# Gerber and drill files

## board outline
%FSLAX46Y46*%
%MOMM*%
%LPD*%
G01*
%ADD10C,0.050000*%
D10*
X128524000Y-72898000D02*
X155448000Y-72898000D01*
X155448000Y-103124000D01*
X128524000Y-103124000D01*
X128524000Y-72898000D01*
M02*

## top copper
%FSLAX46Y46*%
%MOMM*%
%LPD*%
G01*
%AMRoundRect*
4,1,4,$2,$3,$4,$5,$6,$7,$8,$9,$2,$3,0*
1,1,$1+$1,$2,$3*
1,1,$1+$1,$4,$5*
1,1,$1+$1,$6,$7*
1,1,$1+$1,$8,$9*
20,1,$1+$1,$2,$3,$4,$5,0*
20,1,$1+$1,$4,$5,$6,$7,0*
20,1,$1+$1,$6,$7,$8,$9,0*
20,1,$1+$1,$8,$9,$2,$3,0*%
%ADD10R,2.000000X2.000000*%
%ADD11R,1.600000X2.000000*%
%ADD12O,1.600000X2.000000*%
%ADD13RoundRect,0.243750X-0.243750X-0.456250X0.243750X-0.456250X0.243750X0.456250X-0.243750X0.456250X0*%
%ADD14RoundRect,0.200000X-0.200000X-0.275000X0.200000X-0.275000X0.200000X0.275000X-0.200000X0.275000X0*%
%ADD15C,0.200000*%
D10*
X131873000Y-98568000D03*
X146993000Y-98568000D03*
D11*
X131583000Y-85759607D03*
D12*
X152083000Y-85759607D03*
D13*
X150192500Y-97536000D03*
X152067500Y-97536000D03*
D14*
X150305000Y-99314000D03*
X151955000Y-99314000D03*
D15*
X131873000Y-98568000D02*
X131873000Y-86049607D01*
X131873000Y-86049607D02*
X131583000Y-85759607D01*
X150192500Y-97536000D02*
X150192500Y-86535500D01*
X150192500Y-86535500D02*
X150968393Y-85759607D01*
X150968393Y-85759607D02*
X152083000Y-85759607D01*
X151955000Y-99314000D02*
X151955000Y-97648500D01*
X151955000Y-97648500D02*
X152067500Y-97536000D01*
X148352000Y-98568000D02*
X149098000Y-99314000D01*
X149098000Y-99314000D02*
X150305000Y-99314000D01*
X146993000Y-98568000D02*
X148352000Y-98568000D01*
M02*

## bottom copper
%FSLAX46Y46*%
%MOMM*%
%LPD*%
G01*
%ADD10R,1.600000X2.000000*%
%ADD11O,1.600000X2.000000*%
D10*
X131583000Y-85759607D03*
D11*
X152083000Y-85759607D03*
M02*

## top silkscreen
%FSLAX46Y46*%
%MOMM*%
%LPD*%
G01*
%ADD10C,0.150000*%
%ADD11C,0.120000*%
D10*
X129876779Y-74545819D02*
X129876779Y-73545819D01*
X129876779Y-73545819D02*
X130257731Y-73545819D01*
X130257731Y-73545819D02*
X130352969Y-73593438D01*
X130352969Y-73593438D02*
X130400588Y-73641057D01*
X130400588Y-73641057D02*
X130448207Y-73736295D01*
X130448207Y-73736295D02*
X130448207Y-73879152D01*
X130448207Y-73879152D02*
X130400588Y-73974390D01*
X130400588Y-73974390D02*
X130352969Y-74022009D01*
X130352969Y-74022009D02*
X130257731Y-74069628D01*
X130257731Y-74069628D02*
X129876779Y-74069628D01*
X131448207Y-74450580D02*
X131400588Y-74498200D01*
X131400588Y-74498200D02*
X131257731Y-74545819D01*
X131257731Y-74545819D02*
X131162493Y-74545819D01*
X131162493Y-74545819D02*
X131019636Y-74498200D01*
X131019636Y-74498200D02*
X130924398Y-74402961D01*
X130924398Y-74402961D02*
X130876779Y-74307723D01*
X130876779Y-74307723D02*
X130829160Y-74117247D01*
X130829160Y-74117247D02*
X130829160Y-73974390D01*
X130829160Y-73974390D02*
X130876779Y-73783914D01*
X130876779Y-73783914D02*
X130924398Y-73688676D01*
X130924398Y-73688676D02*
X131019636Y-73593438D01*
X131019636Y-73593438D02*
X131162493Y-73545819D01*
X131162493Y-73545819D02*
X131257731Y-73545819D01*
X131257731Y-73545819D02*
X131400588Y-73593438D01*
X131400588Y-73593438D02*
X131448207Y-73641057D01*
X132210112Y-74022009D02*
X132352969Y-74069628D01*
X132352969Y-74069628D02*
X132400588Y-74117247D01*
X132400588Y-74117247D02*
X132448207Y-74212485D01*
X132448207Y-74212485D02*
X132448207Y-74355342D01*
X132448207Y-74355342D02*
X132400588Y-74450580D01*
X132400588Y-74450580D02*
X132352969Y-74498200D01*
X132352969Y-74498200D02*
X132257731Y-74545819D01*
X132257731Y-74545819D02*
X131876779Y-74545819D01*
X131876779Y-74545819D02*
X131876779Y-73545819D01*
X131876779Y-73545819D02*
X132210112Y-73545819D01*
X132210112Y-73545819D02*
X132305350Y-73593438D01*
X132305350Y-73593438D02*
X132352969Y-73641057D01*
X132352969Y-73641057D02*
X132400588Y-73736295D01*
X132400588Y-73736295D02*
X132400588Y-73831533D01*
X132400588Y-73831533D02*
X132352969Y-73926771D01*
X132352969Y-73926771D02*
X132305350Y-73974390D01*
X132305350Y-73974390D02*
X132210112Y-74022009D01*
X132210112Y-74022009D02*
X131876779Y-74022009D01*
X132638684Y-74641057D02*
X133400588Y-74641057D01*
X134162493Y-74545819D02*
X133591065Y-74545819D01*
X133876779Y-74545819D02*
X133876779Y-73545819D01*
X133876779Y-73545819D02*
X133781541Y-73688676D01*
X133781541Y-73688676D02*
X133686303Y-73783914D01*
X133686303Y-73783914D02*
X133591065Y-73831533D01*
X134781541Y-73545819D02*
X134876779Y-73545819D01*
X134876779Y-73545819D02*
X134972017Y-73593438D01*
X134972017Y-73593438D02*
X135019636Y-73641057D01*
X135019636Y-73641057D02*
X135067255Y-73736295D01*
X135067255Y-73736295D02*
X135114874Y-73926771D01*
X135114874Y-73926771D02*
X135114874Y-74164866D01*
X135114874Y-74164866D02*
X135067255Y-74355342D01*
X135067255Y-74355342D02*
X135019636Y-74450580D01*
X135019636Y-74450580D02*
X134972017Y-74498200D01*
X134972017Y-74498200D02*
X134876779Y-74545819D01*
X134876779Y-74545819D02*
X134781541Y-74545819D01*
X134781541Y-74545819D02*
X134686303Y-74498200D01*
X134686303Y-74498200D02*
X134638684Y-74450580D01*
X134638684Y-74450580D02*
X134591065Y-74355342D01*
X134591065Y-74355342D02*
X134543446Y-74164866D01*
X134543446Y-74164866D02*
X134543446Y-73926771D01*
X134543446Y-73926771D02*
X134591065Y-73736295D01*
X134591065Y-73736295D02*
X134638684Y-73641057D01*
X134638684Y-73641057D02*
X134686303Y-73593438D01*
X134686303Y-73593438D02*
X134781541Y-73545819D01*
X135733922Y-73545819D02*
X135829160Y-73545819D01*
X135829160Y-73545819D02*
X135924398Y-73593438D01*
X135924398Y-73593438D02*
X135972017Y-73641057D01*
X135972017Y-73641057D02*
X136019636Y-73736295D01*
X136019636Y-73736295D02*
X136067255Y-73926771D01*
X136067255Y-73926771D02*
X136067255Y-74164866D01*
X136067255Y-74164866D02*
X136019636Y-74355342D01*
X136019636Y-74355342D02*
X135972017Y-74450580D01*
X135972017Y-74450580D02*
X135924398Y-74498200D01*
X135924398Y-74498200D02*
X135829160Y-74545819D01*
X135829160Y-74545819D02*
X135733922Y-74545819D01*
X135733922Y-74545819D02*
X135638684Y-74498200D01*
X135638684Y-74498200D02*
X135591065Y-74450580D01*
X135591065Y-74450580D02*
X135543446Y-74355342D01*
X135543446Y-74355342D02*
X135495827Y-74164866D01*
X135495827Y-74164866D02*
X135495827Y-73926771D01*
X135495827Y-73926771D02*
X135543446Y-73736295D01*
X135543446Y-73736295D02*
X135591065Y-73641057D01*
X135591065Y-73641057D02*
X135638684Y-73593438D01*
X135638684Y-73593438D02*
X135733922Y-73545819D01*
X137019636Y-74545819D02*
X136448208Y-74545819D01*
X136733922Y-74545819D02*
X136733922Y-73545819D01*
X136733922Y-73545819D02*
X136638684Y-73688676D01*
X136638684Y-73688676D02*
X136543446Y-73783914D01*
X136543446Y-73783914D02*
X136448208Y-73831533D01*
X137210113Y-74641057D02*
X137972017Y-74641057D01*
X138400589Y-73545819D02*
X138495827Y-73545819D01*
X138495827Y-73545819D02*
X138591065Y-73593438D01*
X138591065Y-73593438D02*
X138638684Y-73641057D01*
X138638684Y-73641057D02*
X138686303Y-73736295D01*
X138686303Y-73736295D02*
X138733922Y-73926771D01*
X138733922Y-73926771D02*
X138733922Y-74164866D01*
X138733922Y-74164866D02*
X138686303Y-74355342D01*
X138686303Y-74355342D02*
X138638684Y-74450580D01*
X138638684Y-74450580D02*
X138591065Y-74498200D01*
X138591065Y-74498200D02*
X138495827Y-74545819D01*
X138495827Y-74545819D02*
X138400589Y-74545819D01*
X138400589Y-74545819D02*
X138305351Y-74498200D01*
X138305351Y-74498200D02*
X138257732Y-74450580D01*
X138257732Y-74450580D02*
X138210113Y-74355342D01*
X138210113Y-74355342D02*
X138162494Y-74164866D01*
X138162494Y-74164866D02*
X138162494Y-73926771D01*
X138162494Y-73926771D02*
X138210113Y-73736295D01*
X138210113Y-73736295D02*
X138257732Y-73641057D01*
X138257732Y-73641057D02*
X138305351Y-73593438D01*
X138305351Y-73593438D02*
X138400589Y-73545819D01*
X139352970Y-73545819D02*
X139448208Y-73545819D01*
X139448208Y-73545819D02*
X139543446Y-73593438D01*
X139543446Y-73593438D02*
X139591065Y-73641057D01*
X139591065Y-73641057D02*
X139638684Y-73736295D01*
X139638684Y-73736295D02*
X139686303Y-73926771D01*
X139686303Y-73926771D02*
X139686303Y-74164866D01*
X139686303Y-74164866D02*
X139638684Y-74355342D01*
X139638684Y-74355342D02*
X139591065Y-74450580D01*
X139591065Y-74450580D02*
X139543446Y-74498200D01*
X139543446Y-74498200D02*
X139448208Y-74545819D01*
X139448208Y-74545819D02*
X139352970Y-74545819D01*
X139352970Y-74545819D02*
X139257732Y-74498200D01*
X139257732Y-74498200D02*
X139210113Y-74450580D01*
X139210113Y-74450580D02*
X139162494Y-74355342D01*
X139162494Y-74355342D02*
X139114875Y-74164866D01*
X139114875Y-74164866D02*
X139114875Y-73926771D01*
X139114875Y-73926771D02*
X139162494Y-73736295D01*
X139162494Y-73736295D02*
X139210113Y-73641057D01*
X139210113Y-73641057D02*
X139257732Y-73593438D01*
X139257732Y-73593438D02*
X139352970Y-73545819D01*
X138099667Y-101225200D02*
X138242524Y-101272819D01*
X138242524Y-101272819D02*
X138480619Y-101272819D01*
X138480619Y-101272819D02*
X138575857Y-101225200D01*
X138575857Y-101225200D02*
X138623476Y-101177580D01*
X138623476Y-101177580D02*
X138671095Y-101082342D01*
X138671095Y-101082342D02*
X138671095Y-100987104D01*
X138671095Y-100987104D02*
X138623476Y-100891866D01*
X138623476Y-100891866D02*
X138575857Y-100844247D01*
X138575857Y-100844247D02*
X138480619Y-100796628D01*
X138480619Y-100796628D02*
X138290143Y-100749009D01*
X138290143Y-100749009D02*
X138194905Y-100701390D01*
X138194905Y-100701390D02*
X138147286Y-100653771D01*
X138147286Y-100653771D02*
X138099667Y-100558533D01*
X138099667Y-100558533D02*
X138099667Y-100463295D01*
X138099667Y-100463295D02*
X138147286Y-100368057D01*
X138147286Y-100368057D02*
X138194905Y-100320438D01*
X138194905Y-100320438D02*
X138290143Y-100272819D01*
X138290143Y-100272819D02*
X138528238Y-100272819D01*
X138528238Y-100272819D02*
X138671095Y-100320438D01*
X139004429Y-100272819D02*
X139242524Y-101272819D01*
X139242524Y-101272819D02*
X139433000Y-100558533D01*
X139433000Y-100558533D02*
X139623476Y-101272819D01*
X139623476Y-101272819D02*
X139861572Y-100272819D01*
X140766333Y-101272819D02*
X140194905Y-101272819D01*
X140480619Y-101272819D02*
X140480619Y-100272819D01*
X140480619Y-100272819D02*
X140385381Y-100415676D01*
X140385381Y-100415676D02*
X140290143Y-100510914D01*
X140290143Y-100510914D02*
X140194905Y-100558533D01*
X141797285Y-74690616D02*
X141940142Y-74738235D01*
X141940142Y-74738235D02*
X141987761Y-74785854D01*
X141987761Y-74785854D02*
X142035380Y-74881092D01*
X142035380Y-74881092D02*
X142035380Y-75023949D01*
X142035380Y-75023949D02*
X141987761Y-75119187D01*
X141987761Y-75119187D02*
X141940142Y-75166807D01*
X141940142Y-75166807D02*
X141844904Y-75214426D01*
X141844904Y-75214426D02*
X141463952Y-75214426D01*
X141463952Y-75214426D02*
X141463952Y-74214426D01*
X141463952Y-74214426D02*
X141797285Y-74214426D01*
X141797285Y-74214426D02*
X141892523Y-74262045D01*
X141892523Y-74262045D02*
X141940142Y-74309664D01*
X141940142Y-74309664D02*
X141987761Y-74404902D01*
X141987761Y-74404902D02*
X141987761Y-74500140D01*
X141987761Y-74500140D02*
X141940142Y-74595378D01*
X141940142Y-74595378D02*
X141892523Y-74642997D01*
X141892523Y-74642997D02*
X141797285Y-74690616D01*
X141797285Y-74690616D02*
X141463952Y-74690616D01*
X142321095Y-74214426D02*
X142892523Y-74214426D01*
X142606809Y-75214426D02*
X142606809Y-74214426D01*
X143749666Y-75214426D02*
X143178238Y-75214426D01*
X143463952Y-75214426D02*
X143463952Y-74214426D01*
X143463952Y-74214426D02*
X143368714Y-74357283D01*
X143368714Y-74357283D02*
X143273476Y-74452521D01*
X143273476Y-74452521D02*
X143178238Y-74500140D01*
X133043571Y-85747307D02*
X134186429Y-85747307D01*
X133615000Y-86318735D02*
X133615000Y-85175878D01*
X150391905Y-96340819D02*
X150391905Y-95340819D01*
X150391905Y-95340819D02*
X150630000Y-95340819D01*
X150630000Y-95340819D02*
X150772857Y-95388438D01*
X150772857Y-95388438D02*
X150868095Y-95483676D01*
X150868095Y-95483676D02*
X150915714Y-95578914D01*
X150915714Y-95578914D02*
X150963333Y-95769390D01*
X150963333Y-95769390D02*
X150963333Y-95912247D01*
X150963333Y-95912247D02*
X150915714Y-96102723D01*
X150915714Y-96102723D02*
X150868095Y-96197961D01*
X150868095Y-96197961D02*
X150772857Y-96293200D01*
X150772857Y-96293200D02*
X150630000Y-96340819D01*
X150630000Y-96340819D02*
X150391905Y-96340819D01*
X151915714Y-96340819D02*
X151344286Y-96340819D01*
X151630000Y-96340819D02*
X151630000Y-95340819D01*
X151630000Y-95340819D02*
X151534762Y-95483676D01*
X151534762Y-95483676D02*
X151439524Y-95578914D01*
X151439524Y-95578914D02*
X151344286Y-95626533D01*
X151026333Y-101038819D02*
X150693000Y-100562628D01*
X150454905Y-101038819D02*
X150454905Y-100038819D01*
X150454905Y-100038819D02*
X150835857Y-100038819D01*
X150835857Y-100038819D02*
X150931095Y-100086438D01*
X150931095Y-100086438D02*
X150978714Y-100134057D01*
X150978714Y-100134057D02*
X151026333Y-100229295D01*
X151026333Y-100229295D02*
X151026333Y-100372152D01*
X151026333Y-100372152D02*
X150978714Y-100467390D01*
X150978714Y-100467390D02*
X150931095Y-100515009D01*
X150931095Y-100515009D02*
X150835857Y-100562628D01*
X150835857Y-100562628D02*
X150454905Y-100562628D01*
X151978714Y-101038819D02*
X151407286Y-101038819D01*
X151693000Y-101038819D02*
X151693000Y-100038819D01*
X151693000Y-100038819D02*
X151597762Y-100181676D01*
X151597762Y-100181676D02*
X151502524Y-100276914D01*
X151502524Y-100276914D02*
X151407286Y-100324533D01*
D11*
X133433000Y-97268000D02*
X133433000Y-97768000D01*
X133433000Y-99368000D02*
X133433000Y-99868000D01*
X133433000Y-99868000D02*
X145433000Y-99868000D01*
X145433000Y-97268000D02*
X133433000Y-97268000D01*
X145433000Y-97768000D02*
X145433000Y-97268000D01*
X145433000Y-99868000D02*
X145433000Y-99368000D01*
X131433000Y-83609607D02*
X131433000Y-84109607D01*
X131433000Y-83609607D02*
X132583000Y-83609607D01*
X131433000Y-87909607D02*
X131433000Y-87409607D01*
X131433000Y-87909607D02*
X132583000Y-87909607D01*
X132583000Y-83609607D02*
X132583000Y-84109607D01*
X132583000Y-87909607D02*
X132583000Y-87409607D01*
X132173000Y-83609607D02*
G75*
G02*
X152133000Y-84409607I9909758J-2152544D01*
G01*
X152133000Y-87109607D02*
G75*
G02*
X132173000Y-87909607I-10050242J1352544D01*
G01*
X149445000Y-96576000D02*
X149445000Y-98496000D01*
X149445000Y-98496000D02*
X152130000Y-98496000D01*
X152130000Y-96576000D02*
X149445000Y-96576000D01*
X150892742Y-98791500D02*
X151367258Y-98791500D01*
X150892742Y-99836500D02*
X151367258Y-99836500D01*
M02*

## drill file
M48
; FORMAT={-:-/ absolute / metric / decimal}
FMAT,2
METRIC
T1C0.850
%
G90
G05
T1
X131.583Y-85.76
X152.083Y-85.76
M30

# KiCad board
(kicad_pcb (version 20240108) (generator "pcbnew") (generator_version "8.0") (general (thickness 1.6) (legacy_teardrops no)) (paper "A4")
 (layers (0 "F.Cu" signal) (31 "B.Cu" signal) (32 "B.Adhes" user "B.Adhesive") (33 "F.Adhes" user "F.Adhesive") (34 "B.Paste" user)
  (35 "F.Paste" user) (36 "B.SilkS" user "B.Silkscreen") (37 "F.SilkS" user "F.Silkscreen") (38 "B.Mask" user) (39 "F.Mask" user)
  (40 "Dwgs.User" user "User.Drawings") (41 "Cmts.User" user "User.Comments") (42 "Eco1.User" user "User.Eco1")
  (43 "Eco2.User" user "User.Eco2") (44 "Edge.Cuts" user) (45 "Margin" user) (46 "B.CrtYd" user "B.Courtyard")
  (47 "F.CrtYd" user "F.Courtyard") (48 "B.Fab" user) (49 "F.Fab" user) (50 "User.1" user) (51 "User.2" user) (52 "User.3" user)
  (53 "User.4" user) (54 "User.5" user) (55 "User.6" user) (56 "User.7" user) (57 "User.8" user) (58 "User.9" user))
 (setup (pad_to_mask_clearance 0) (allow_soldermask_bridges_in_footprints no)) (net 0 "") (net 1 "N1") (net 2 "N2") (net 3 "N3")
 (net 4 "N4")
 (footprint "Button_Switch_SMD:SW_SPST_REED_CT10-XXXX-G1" (layer "F.Cu") (at 139.433 98.568)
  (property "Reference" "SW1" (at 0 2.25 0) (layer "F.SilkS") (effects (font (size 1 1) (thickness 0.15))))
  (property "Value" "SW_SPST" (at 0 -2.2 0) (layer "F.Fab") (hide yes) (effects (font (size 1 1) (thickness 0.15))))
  (fp_line (start -6 -1.3) (end -6 -0.8) (stroke (width 0.12) (type solid)) (layer "F.SilkS"))
  (fp_line (start -6 0.8) (end -6 1.3) (stroke (width 0.12) (type solid)) (layer "F.SilkS"))
  (fp_line (start -6 1.3) (end 6 1.3) (stroke (width 0.12) (type solid)) (layer "F.SilkS"))
  (fp_line (start 6 -1.3) (end -6 -1.3) (stroke (width 0.12) (type solid)) (layer "F.SilkS"))
  (fp_line (start 6 -0.8) (end 6 -1.3) (stroke (width 0.12) (type solid)) (layer "F.SilkS"))
  (fp_line (start 6 1.3) (end 6 0.8) (stroke (width 0.12) (type solid)) (layer "F.SilkS"))
  (pad "1" smd rect (at -7.56 0) (size 2 2) (layers "F.Cu" "F.Paste" "F.Mask") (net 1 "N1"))
  (pad "2" smd rect (at 7.56 0) (size 2 2) (layers "F.Cu" "F.Paste" "F.Mask") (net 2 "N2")))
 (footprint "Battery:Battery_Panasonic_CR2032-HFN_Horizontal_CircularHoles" (layer "F.Cu") (at 131.583 85.759607)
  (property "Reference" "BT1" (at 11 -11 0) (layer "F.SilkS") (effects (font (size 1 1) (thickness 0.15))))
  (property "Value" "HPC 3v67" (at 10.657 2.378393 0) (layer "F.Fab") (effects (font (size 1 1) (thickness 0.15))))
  (fp_line (start -0.15 -2.15) (end -0.15 -1.65) (stroke (width 0.12) (type default)) (layer "F.SilkS"))
  (fp_line (start -0.15 -2.15) (end 1 -2.15) (stroke (width 0.12) (type default)) (layer "F.SilkS"))
  (fp_line (start -0.15 2.15) (end -0.15 1.65) (stroke (width 0.12) (type default)) (layer "F.SilkS"))
  (fp_line (start -0.15 2.15) (end 1 2.15) (stroke (width 0.12) (type default)) (layer "F.SilkS"))
  (fp_line (start 1 -2.15) (end 1 -1.65) (stroke (width 0.12) (type default)) (layer "F.SilkS"))
  (fp_line (start 1 2.15) (end 1 1.65) (stroke (width 0.12) (type default)) (layer "F.SilkS"))
  (fp_arc (start 0.59 -2.15) (mid 10.905879 -10.130166) (end 20.55 -1.35) (stroke (width 0.12) (type default)) (layer "F.SilkS"))
  (fp_arc (start 20.55 1.35) (mid 10.905879 10.130166) (end 0.59 2.15) (stroke (width 0.12) (type default)) (layer "F.SilkS"))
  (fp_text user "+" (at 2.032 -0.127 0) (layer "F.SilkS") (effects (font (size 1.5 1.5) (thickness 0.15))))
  (pad "1" thru_hole rect (at 0 0) (size 1.6 2) (drill 0.85) (layers "*.Cu" "*.Mask") (remove_unused_layers no) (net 1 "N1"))
  (pad "2" thru_hole oval (at 20.5 0) (size 1.6 2) (drill 0.85) (layers "*.Cu" "*.Mask") (remove_unused_layers no) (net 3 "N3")))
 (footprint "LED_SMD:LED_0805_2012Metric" (layer "F.Cu") (at 151.13 97.536)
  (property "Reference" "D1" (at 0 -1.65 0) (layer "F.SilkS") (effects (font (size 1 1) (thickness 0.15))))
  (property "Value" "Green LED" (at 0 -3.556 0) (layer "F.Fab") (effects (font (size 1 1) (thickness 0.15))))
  (fp_line (start -1.685 -0.96) (end -1.685 0.96) (stroke (width 0.12) (type solid)) (layer "F.SilkS"))
  (fp_line (start -1.685 0.96) (end 1 0.96) (stroke (width 0.12) (type solid)) (layer "F.SilkS"))
  (fp_line (start 1 -0.96) (end -1.685 -0.96) (stroke (width 0.12) (type solid)) (layer "F.SilkS"))
  (pad "1" smd roundrect (at -0.9375 0) (size 0.975 1.4) (layers "F.Cu" "F.Paste" "F.Mask") (roundrect_rratio 0.25) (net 3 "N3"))
  (pad "2" smd roundrect (at 0.9375 0) (size 0.975 1.4) (layers "F.Cu" "F.Paste" "F.Mask") (roundrect_rratio 0.25) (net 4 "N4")))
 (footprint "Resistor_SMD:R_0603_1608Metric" (layer "F.Cu") (at 151.13 99.314)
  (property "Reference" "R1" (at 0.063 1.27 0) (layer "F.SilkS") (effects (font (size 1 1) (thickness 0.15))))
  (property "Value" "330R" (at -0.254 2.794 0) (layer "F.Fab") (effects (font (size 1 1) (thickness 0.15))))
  (fp_line (start -0.237258 -0.5225) (end 0.237258 -0.5225) (stroke (width 0.12) (type solid)) (layer "F.SilkS"))
  (fp_line (start -0.237258 0.5225) (end 0.237258 0.5225) (stroke (width 0.12) (type solid)) (layer "F.SilkS"))
  (pad "1" smd roundrect (at -0.825 0) (size 0.8 0.95) (layers "F.Cu" "F.Paste" "F.Mask") (roundrect_rratio 0.25) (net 2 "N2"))
  (pad "2" smd roundrect (at 0.825 0) (size 0.8 0.95) (layers "F.Cu" "F.Paste" "F.Mask") (roundrect_rratio 0.25) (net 4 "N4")))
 (gr_rect (start 128.524 72.898) (end 155.448 103.124) (stroke (width 0.05) (type default)) (fill none) (layer "Edge.Cuts"))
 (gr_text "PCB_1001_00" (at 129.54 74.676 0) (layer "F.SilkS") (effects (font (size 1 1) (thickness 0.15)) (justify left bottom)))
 (segment (start 131.873 98.568) (end 131.873 86.049607) (width 0.2) (layer "F.Cu") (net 1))
 (segment (start 131.873 86.049607) (end 131.583 85.759607) (width 0.2) (layer "F.Cu") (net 1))
 (segment (start 150.1925 97.536) (end 150.1925 86.5355) (width 0.2) (layer "F.Cu") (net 3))
 (segment (start 150.1925 86.5355) (end 150.968393 85.759607) (width 0.2) (layer "F.Cu") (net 3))
 (segment (start 150.968393 85.759607) (end 152.083 85.759607) (width 0.2) (layer "F.Cu") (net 3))
 (segment (start 151.955 99.314) (end 151.955 97.6485) (width 0.2) (layer "F.Cu") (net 4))
 (segment (start 151.955 97.6485) (end 152.0675 97.536) (width 0.2) (layer "F.Cu") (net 4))
 (segment (start 148.352 98.568) (end 149.098 99.314) (width 0.2) (layer "F.Cu") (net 2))
 (segment (start 149.098 99.314) (end 150.305 99.314) (width 0.2) (layer "F.Cu") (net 2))
 (segment (start 146.993 98.568) (end 148.352 98.568) (width 0.2) (layer "F.Cu") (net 2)))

